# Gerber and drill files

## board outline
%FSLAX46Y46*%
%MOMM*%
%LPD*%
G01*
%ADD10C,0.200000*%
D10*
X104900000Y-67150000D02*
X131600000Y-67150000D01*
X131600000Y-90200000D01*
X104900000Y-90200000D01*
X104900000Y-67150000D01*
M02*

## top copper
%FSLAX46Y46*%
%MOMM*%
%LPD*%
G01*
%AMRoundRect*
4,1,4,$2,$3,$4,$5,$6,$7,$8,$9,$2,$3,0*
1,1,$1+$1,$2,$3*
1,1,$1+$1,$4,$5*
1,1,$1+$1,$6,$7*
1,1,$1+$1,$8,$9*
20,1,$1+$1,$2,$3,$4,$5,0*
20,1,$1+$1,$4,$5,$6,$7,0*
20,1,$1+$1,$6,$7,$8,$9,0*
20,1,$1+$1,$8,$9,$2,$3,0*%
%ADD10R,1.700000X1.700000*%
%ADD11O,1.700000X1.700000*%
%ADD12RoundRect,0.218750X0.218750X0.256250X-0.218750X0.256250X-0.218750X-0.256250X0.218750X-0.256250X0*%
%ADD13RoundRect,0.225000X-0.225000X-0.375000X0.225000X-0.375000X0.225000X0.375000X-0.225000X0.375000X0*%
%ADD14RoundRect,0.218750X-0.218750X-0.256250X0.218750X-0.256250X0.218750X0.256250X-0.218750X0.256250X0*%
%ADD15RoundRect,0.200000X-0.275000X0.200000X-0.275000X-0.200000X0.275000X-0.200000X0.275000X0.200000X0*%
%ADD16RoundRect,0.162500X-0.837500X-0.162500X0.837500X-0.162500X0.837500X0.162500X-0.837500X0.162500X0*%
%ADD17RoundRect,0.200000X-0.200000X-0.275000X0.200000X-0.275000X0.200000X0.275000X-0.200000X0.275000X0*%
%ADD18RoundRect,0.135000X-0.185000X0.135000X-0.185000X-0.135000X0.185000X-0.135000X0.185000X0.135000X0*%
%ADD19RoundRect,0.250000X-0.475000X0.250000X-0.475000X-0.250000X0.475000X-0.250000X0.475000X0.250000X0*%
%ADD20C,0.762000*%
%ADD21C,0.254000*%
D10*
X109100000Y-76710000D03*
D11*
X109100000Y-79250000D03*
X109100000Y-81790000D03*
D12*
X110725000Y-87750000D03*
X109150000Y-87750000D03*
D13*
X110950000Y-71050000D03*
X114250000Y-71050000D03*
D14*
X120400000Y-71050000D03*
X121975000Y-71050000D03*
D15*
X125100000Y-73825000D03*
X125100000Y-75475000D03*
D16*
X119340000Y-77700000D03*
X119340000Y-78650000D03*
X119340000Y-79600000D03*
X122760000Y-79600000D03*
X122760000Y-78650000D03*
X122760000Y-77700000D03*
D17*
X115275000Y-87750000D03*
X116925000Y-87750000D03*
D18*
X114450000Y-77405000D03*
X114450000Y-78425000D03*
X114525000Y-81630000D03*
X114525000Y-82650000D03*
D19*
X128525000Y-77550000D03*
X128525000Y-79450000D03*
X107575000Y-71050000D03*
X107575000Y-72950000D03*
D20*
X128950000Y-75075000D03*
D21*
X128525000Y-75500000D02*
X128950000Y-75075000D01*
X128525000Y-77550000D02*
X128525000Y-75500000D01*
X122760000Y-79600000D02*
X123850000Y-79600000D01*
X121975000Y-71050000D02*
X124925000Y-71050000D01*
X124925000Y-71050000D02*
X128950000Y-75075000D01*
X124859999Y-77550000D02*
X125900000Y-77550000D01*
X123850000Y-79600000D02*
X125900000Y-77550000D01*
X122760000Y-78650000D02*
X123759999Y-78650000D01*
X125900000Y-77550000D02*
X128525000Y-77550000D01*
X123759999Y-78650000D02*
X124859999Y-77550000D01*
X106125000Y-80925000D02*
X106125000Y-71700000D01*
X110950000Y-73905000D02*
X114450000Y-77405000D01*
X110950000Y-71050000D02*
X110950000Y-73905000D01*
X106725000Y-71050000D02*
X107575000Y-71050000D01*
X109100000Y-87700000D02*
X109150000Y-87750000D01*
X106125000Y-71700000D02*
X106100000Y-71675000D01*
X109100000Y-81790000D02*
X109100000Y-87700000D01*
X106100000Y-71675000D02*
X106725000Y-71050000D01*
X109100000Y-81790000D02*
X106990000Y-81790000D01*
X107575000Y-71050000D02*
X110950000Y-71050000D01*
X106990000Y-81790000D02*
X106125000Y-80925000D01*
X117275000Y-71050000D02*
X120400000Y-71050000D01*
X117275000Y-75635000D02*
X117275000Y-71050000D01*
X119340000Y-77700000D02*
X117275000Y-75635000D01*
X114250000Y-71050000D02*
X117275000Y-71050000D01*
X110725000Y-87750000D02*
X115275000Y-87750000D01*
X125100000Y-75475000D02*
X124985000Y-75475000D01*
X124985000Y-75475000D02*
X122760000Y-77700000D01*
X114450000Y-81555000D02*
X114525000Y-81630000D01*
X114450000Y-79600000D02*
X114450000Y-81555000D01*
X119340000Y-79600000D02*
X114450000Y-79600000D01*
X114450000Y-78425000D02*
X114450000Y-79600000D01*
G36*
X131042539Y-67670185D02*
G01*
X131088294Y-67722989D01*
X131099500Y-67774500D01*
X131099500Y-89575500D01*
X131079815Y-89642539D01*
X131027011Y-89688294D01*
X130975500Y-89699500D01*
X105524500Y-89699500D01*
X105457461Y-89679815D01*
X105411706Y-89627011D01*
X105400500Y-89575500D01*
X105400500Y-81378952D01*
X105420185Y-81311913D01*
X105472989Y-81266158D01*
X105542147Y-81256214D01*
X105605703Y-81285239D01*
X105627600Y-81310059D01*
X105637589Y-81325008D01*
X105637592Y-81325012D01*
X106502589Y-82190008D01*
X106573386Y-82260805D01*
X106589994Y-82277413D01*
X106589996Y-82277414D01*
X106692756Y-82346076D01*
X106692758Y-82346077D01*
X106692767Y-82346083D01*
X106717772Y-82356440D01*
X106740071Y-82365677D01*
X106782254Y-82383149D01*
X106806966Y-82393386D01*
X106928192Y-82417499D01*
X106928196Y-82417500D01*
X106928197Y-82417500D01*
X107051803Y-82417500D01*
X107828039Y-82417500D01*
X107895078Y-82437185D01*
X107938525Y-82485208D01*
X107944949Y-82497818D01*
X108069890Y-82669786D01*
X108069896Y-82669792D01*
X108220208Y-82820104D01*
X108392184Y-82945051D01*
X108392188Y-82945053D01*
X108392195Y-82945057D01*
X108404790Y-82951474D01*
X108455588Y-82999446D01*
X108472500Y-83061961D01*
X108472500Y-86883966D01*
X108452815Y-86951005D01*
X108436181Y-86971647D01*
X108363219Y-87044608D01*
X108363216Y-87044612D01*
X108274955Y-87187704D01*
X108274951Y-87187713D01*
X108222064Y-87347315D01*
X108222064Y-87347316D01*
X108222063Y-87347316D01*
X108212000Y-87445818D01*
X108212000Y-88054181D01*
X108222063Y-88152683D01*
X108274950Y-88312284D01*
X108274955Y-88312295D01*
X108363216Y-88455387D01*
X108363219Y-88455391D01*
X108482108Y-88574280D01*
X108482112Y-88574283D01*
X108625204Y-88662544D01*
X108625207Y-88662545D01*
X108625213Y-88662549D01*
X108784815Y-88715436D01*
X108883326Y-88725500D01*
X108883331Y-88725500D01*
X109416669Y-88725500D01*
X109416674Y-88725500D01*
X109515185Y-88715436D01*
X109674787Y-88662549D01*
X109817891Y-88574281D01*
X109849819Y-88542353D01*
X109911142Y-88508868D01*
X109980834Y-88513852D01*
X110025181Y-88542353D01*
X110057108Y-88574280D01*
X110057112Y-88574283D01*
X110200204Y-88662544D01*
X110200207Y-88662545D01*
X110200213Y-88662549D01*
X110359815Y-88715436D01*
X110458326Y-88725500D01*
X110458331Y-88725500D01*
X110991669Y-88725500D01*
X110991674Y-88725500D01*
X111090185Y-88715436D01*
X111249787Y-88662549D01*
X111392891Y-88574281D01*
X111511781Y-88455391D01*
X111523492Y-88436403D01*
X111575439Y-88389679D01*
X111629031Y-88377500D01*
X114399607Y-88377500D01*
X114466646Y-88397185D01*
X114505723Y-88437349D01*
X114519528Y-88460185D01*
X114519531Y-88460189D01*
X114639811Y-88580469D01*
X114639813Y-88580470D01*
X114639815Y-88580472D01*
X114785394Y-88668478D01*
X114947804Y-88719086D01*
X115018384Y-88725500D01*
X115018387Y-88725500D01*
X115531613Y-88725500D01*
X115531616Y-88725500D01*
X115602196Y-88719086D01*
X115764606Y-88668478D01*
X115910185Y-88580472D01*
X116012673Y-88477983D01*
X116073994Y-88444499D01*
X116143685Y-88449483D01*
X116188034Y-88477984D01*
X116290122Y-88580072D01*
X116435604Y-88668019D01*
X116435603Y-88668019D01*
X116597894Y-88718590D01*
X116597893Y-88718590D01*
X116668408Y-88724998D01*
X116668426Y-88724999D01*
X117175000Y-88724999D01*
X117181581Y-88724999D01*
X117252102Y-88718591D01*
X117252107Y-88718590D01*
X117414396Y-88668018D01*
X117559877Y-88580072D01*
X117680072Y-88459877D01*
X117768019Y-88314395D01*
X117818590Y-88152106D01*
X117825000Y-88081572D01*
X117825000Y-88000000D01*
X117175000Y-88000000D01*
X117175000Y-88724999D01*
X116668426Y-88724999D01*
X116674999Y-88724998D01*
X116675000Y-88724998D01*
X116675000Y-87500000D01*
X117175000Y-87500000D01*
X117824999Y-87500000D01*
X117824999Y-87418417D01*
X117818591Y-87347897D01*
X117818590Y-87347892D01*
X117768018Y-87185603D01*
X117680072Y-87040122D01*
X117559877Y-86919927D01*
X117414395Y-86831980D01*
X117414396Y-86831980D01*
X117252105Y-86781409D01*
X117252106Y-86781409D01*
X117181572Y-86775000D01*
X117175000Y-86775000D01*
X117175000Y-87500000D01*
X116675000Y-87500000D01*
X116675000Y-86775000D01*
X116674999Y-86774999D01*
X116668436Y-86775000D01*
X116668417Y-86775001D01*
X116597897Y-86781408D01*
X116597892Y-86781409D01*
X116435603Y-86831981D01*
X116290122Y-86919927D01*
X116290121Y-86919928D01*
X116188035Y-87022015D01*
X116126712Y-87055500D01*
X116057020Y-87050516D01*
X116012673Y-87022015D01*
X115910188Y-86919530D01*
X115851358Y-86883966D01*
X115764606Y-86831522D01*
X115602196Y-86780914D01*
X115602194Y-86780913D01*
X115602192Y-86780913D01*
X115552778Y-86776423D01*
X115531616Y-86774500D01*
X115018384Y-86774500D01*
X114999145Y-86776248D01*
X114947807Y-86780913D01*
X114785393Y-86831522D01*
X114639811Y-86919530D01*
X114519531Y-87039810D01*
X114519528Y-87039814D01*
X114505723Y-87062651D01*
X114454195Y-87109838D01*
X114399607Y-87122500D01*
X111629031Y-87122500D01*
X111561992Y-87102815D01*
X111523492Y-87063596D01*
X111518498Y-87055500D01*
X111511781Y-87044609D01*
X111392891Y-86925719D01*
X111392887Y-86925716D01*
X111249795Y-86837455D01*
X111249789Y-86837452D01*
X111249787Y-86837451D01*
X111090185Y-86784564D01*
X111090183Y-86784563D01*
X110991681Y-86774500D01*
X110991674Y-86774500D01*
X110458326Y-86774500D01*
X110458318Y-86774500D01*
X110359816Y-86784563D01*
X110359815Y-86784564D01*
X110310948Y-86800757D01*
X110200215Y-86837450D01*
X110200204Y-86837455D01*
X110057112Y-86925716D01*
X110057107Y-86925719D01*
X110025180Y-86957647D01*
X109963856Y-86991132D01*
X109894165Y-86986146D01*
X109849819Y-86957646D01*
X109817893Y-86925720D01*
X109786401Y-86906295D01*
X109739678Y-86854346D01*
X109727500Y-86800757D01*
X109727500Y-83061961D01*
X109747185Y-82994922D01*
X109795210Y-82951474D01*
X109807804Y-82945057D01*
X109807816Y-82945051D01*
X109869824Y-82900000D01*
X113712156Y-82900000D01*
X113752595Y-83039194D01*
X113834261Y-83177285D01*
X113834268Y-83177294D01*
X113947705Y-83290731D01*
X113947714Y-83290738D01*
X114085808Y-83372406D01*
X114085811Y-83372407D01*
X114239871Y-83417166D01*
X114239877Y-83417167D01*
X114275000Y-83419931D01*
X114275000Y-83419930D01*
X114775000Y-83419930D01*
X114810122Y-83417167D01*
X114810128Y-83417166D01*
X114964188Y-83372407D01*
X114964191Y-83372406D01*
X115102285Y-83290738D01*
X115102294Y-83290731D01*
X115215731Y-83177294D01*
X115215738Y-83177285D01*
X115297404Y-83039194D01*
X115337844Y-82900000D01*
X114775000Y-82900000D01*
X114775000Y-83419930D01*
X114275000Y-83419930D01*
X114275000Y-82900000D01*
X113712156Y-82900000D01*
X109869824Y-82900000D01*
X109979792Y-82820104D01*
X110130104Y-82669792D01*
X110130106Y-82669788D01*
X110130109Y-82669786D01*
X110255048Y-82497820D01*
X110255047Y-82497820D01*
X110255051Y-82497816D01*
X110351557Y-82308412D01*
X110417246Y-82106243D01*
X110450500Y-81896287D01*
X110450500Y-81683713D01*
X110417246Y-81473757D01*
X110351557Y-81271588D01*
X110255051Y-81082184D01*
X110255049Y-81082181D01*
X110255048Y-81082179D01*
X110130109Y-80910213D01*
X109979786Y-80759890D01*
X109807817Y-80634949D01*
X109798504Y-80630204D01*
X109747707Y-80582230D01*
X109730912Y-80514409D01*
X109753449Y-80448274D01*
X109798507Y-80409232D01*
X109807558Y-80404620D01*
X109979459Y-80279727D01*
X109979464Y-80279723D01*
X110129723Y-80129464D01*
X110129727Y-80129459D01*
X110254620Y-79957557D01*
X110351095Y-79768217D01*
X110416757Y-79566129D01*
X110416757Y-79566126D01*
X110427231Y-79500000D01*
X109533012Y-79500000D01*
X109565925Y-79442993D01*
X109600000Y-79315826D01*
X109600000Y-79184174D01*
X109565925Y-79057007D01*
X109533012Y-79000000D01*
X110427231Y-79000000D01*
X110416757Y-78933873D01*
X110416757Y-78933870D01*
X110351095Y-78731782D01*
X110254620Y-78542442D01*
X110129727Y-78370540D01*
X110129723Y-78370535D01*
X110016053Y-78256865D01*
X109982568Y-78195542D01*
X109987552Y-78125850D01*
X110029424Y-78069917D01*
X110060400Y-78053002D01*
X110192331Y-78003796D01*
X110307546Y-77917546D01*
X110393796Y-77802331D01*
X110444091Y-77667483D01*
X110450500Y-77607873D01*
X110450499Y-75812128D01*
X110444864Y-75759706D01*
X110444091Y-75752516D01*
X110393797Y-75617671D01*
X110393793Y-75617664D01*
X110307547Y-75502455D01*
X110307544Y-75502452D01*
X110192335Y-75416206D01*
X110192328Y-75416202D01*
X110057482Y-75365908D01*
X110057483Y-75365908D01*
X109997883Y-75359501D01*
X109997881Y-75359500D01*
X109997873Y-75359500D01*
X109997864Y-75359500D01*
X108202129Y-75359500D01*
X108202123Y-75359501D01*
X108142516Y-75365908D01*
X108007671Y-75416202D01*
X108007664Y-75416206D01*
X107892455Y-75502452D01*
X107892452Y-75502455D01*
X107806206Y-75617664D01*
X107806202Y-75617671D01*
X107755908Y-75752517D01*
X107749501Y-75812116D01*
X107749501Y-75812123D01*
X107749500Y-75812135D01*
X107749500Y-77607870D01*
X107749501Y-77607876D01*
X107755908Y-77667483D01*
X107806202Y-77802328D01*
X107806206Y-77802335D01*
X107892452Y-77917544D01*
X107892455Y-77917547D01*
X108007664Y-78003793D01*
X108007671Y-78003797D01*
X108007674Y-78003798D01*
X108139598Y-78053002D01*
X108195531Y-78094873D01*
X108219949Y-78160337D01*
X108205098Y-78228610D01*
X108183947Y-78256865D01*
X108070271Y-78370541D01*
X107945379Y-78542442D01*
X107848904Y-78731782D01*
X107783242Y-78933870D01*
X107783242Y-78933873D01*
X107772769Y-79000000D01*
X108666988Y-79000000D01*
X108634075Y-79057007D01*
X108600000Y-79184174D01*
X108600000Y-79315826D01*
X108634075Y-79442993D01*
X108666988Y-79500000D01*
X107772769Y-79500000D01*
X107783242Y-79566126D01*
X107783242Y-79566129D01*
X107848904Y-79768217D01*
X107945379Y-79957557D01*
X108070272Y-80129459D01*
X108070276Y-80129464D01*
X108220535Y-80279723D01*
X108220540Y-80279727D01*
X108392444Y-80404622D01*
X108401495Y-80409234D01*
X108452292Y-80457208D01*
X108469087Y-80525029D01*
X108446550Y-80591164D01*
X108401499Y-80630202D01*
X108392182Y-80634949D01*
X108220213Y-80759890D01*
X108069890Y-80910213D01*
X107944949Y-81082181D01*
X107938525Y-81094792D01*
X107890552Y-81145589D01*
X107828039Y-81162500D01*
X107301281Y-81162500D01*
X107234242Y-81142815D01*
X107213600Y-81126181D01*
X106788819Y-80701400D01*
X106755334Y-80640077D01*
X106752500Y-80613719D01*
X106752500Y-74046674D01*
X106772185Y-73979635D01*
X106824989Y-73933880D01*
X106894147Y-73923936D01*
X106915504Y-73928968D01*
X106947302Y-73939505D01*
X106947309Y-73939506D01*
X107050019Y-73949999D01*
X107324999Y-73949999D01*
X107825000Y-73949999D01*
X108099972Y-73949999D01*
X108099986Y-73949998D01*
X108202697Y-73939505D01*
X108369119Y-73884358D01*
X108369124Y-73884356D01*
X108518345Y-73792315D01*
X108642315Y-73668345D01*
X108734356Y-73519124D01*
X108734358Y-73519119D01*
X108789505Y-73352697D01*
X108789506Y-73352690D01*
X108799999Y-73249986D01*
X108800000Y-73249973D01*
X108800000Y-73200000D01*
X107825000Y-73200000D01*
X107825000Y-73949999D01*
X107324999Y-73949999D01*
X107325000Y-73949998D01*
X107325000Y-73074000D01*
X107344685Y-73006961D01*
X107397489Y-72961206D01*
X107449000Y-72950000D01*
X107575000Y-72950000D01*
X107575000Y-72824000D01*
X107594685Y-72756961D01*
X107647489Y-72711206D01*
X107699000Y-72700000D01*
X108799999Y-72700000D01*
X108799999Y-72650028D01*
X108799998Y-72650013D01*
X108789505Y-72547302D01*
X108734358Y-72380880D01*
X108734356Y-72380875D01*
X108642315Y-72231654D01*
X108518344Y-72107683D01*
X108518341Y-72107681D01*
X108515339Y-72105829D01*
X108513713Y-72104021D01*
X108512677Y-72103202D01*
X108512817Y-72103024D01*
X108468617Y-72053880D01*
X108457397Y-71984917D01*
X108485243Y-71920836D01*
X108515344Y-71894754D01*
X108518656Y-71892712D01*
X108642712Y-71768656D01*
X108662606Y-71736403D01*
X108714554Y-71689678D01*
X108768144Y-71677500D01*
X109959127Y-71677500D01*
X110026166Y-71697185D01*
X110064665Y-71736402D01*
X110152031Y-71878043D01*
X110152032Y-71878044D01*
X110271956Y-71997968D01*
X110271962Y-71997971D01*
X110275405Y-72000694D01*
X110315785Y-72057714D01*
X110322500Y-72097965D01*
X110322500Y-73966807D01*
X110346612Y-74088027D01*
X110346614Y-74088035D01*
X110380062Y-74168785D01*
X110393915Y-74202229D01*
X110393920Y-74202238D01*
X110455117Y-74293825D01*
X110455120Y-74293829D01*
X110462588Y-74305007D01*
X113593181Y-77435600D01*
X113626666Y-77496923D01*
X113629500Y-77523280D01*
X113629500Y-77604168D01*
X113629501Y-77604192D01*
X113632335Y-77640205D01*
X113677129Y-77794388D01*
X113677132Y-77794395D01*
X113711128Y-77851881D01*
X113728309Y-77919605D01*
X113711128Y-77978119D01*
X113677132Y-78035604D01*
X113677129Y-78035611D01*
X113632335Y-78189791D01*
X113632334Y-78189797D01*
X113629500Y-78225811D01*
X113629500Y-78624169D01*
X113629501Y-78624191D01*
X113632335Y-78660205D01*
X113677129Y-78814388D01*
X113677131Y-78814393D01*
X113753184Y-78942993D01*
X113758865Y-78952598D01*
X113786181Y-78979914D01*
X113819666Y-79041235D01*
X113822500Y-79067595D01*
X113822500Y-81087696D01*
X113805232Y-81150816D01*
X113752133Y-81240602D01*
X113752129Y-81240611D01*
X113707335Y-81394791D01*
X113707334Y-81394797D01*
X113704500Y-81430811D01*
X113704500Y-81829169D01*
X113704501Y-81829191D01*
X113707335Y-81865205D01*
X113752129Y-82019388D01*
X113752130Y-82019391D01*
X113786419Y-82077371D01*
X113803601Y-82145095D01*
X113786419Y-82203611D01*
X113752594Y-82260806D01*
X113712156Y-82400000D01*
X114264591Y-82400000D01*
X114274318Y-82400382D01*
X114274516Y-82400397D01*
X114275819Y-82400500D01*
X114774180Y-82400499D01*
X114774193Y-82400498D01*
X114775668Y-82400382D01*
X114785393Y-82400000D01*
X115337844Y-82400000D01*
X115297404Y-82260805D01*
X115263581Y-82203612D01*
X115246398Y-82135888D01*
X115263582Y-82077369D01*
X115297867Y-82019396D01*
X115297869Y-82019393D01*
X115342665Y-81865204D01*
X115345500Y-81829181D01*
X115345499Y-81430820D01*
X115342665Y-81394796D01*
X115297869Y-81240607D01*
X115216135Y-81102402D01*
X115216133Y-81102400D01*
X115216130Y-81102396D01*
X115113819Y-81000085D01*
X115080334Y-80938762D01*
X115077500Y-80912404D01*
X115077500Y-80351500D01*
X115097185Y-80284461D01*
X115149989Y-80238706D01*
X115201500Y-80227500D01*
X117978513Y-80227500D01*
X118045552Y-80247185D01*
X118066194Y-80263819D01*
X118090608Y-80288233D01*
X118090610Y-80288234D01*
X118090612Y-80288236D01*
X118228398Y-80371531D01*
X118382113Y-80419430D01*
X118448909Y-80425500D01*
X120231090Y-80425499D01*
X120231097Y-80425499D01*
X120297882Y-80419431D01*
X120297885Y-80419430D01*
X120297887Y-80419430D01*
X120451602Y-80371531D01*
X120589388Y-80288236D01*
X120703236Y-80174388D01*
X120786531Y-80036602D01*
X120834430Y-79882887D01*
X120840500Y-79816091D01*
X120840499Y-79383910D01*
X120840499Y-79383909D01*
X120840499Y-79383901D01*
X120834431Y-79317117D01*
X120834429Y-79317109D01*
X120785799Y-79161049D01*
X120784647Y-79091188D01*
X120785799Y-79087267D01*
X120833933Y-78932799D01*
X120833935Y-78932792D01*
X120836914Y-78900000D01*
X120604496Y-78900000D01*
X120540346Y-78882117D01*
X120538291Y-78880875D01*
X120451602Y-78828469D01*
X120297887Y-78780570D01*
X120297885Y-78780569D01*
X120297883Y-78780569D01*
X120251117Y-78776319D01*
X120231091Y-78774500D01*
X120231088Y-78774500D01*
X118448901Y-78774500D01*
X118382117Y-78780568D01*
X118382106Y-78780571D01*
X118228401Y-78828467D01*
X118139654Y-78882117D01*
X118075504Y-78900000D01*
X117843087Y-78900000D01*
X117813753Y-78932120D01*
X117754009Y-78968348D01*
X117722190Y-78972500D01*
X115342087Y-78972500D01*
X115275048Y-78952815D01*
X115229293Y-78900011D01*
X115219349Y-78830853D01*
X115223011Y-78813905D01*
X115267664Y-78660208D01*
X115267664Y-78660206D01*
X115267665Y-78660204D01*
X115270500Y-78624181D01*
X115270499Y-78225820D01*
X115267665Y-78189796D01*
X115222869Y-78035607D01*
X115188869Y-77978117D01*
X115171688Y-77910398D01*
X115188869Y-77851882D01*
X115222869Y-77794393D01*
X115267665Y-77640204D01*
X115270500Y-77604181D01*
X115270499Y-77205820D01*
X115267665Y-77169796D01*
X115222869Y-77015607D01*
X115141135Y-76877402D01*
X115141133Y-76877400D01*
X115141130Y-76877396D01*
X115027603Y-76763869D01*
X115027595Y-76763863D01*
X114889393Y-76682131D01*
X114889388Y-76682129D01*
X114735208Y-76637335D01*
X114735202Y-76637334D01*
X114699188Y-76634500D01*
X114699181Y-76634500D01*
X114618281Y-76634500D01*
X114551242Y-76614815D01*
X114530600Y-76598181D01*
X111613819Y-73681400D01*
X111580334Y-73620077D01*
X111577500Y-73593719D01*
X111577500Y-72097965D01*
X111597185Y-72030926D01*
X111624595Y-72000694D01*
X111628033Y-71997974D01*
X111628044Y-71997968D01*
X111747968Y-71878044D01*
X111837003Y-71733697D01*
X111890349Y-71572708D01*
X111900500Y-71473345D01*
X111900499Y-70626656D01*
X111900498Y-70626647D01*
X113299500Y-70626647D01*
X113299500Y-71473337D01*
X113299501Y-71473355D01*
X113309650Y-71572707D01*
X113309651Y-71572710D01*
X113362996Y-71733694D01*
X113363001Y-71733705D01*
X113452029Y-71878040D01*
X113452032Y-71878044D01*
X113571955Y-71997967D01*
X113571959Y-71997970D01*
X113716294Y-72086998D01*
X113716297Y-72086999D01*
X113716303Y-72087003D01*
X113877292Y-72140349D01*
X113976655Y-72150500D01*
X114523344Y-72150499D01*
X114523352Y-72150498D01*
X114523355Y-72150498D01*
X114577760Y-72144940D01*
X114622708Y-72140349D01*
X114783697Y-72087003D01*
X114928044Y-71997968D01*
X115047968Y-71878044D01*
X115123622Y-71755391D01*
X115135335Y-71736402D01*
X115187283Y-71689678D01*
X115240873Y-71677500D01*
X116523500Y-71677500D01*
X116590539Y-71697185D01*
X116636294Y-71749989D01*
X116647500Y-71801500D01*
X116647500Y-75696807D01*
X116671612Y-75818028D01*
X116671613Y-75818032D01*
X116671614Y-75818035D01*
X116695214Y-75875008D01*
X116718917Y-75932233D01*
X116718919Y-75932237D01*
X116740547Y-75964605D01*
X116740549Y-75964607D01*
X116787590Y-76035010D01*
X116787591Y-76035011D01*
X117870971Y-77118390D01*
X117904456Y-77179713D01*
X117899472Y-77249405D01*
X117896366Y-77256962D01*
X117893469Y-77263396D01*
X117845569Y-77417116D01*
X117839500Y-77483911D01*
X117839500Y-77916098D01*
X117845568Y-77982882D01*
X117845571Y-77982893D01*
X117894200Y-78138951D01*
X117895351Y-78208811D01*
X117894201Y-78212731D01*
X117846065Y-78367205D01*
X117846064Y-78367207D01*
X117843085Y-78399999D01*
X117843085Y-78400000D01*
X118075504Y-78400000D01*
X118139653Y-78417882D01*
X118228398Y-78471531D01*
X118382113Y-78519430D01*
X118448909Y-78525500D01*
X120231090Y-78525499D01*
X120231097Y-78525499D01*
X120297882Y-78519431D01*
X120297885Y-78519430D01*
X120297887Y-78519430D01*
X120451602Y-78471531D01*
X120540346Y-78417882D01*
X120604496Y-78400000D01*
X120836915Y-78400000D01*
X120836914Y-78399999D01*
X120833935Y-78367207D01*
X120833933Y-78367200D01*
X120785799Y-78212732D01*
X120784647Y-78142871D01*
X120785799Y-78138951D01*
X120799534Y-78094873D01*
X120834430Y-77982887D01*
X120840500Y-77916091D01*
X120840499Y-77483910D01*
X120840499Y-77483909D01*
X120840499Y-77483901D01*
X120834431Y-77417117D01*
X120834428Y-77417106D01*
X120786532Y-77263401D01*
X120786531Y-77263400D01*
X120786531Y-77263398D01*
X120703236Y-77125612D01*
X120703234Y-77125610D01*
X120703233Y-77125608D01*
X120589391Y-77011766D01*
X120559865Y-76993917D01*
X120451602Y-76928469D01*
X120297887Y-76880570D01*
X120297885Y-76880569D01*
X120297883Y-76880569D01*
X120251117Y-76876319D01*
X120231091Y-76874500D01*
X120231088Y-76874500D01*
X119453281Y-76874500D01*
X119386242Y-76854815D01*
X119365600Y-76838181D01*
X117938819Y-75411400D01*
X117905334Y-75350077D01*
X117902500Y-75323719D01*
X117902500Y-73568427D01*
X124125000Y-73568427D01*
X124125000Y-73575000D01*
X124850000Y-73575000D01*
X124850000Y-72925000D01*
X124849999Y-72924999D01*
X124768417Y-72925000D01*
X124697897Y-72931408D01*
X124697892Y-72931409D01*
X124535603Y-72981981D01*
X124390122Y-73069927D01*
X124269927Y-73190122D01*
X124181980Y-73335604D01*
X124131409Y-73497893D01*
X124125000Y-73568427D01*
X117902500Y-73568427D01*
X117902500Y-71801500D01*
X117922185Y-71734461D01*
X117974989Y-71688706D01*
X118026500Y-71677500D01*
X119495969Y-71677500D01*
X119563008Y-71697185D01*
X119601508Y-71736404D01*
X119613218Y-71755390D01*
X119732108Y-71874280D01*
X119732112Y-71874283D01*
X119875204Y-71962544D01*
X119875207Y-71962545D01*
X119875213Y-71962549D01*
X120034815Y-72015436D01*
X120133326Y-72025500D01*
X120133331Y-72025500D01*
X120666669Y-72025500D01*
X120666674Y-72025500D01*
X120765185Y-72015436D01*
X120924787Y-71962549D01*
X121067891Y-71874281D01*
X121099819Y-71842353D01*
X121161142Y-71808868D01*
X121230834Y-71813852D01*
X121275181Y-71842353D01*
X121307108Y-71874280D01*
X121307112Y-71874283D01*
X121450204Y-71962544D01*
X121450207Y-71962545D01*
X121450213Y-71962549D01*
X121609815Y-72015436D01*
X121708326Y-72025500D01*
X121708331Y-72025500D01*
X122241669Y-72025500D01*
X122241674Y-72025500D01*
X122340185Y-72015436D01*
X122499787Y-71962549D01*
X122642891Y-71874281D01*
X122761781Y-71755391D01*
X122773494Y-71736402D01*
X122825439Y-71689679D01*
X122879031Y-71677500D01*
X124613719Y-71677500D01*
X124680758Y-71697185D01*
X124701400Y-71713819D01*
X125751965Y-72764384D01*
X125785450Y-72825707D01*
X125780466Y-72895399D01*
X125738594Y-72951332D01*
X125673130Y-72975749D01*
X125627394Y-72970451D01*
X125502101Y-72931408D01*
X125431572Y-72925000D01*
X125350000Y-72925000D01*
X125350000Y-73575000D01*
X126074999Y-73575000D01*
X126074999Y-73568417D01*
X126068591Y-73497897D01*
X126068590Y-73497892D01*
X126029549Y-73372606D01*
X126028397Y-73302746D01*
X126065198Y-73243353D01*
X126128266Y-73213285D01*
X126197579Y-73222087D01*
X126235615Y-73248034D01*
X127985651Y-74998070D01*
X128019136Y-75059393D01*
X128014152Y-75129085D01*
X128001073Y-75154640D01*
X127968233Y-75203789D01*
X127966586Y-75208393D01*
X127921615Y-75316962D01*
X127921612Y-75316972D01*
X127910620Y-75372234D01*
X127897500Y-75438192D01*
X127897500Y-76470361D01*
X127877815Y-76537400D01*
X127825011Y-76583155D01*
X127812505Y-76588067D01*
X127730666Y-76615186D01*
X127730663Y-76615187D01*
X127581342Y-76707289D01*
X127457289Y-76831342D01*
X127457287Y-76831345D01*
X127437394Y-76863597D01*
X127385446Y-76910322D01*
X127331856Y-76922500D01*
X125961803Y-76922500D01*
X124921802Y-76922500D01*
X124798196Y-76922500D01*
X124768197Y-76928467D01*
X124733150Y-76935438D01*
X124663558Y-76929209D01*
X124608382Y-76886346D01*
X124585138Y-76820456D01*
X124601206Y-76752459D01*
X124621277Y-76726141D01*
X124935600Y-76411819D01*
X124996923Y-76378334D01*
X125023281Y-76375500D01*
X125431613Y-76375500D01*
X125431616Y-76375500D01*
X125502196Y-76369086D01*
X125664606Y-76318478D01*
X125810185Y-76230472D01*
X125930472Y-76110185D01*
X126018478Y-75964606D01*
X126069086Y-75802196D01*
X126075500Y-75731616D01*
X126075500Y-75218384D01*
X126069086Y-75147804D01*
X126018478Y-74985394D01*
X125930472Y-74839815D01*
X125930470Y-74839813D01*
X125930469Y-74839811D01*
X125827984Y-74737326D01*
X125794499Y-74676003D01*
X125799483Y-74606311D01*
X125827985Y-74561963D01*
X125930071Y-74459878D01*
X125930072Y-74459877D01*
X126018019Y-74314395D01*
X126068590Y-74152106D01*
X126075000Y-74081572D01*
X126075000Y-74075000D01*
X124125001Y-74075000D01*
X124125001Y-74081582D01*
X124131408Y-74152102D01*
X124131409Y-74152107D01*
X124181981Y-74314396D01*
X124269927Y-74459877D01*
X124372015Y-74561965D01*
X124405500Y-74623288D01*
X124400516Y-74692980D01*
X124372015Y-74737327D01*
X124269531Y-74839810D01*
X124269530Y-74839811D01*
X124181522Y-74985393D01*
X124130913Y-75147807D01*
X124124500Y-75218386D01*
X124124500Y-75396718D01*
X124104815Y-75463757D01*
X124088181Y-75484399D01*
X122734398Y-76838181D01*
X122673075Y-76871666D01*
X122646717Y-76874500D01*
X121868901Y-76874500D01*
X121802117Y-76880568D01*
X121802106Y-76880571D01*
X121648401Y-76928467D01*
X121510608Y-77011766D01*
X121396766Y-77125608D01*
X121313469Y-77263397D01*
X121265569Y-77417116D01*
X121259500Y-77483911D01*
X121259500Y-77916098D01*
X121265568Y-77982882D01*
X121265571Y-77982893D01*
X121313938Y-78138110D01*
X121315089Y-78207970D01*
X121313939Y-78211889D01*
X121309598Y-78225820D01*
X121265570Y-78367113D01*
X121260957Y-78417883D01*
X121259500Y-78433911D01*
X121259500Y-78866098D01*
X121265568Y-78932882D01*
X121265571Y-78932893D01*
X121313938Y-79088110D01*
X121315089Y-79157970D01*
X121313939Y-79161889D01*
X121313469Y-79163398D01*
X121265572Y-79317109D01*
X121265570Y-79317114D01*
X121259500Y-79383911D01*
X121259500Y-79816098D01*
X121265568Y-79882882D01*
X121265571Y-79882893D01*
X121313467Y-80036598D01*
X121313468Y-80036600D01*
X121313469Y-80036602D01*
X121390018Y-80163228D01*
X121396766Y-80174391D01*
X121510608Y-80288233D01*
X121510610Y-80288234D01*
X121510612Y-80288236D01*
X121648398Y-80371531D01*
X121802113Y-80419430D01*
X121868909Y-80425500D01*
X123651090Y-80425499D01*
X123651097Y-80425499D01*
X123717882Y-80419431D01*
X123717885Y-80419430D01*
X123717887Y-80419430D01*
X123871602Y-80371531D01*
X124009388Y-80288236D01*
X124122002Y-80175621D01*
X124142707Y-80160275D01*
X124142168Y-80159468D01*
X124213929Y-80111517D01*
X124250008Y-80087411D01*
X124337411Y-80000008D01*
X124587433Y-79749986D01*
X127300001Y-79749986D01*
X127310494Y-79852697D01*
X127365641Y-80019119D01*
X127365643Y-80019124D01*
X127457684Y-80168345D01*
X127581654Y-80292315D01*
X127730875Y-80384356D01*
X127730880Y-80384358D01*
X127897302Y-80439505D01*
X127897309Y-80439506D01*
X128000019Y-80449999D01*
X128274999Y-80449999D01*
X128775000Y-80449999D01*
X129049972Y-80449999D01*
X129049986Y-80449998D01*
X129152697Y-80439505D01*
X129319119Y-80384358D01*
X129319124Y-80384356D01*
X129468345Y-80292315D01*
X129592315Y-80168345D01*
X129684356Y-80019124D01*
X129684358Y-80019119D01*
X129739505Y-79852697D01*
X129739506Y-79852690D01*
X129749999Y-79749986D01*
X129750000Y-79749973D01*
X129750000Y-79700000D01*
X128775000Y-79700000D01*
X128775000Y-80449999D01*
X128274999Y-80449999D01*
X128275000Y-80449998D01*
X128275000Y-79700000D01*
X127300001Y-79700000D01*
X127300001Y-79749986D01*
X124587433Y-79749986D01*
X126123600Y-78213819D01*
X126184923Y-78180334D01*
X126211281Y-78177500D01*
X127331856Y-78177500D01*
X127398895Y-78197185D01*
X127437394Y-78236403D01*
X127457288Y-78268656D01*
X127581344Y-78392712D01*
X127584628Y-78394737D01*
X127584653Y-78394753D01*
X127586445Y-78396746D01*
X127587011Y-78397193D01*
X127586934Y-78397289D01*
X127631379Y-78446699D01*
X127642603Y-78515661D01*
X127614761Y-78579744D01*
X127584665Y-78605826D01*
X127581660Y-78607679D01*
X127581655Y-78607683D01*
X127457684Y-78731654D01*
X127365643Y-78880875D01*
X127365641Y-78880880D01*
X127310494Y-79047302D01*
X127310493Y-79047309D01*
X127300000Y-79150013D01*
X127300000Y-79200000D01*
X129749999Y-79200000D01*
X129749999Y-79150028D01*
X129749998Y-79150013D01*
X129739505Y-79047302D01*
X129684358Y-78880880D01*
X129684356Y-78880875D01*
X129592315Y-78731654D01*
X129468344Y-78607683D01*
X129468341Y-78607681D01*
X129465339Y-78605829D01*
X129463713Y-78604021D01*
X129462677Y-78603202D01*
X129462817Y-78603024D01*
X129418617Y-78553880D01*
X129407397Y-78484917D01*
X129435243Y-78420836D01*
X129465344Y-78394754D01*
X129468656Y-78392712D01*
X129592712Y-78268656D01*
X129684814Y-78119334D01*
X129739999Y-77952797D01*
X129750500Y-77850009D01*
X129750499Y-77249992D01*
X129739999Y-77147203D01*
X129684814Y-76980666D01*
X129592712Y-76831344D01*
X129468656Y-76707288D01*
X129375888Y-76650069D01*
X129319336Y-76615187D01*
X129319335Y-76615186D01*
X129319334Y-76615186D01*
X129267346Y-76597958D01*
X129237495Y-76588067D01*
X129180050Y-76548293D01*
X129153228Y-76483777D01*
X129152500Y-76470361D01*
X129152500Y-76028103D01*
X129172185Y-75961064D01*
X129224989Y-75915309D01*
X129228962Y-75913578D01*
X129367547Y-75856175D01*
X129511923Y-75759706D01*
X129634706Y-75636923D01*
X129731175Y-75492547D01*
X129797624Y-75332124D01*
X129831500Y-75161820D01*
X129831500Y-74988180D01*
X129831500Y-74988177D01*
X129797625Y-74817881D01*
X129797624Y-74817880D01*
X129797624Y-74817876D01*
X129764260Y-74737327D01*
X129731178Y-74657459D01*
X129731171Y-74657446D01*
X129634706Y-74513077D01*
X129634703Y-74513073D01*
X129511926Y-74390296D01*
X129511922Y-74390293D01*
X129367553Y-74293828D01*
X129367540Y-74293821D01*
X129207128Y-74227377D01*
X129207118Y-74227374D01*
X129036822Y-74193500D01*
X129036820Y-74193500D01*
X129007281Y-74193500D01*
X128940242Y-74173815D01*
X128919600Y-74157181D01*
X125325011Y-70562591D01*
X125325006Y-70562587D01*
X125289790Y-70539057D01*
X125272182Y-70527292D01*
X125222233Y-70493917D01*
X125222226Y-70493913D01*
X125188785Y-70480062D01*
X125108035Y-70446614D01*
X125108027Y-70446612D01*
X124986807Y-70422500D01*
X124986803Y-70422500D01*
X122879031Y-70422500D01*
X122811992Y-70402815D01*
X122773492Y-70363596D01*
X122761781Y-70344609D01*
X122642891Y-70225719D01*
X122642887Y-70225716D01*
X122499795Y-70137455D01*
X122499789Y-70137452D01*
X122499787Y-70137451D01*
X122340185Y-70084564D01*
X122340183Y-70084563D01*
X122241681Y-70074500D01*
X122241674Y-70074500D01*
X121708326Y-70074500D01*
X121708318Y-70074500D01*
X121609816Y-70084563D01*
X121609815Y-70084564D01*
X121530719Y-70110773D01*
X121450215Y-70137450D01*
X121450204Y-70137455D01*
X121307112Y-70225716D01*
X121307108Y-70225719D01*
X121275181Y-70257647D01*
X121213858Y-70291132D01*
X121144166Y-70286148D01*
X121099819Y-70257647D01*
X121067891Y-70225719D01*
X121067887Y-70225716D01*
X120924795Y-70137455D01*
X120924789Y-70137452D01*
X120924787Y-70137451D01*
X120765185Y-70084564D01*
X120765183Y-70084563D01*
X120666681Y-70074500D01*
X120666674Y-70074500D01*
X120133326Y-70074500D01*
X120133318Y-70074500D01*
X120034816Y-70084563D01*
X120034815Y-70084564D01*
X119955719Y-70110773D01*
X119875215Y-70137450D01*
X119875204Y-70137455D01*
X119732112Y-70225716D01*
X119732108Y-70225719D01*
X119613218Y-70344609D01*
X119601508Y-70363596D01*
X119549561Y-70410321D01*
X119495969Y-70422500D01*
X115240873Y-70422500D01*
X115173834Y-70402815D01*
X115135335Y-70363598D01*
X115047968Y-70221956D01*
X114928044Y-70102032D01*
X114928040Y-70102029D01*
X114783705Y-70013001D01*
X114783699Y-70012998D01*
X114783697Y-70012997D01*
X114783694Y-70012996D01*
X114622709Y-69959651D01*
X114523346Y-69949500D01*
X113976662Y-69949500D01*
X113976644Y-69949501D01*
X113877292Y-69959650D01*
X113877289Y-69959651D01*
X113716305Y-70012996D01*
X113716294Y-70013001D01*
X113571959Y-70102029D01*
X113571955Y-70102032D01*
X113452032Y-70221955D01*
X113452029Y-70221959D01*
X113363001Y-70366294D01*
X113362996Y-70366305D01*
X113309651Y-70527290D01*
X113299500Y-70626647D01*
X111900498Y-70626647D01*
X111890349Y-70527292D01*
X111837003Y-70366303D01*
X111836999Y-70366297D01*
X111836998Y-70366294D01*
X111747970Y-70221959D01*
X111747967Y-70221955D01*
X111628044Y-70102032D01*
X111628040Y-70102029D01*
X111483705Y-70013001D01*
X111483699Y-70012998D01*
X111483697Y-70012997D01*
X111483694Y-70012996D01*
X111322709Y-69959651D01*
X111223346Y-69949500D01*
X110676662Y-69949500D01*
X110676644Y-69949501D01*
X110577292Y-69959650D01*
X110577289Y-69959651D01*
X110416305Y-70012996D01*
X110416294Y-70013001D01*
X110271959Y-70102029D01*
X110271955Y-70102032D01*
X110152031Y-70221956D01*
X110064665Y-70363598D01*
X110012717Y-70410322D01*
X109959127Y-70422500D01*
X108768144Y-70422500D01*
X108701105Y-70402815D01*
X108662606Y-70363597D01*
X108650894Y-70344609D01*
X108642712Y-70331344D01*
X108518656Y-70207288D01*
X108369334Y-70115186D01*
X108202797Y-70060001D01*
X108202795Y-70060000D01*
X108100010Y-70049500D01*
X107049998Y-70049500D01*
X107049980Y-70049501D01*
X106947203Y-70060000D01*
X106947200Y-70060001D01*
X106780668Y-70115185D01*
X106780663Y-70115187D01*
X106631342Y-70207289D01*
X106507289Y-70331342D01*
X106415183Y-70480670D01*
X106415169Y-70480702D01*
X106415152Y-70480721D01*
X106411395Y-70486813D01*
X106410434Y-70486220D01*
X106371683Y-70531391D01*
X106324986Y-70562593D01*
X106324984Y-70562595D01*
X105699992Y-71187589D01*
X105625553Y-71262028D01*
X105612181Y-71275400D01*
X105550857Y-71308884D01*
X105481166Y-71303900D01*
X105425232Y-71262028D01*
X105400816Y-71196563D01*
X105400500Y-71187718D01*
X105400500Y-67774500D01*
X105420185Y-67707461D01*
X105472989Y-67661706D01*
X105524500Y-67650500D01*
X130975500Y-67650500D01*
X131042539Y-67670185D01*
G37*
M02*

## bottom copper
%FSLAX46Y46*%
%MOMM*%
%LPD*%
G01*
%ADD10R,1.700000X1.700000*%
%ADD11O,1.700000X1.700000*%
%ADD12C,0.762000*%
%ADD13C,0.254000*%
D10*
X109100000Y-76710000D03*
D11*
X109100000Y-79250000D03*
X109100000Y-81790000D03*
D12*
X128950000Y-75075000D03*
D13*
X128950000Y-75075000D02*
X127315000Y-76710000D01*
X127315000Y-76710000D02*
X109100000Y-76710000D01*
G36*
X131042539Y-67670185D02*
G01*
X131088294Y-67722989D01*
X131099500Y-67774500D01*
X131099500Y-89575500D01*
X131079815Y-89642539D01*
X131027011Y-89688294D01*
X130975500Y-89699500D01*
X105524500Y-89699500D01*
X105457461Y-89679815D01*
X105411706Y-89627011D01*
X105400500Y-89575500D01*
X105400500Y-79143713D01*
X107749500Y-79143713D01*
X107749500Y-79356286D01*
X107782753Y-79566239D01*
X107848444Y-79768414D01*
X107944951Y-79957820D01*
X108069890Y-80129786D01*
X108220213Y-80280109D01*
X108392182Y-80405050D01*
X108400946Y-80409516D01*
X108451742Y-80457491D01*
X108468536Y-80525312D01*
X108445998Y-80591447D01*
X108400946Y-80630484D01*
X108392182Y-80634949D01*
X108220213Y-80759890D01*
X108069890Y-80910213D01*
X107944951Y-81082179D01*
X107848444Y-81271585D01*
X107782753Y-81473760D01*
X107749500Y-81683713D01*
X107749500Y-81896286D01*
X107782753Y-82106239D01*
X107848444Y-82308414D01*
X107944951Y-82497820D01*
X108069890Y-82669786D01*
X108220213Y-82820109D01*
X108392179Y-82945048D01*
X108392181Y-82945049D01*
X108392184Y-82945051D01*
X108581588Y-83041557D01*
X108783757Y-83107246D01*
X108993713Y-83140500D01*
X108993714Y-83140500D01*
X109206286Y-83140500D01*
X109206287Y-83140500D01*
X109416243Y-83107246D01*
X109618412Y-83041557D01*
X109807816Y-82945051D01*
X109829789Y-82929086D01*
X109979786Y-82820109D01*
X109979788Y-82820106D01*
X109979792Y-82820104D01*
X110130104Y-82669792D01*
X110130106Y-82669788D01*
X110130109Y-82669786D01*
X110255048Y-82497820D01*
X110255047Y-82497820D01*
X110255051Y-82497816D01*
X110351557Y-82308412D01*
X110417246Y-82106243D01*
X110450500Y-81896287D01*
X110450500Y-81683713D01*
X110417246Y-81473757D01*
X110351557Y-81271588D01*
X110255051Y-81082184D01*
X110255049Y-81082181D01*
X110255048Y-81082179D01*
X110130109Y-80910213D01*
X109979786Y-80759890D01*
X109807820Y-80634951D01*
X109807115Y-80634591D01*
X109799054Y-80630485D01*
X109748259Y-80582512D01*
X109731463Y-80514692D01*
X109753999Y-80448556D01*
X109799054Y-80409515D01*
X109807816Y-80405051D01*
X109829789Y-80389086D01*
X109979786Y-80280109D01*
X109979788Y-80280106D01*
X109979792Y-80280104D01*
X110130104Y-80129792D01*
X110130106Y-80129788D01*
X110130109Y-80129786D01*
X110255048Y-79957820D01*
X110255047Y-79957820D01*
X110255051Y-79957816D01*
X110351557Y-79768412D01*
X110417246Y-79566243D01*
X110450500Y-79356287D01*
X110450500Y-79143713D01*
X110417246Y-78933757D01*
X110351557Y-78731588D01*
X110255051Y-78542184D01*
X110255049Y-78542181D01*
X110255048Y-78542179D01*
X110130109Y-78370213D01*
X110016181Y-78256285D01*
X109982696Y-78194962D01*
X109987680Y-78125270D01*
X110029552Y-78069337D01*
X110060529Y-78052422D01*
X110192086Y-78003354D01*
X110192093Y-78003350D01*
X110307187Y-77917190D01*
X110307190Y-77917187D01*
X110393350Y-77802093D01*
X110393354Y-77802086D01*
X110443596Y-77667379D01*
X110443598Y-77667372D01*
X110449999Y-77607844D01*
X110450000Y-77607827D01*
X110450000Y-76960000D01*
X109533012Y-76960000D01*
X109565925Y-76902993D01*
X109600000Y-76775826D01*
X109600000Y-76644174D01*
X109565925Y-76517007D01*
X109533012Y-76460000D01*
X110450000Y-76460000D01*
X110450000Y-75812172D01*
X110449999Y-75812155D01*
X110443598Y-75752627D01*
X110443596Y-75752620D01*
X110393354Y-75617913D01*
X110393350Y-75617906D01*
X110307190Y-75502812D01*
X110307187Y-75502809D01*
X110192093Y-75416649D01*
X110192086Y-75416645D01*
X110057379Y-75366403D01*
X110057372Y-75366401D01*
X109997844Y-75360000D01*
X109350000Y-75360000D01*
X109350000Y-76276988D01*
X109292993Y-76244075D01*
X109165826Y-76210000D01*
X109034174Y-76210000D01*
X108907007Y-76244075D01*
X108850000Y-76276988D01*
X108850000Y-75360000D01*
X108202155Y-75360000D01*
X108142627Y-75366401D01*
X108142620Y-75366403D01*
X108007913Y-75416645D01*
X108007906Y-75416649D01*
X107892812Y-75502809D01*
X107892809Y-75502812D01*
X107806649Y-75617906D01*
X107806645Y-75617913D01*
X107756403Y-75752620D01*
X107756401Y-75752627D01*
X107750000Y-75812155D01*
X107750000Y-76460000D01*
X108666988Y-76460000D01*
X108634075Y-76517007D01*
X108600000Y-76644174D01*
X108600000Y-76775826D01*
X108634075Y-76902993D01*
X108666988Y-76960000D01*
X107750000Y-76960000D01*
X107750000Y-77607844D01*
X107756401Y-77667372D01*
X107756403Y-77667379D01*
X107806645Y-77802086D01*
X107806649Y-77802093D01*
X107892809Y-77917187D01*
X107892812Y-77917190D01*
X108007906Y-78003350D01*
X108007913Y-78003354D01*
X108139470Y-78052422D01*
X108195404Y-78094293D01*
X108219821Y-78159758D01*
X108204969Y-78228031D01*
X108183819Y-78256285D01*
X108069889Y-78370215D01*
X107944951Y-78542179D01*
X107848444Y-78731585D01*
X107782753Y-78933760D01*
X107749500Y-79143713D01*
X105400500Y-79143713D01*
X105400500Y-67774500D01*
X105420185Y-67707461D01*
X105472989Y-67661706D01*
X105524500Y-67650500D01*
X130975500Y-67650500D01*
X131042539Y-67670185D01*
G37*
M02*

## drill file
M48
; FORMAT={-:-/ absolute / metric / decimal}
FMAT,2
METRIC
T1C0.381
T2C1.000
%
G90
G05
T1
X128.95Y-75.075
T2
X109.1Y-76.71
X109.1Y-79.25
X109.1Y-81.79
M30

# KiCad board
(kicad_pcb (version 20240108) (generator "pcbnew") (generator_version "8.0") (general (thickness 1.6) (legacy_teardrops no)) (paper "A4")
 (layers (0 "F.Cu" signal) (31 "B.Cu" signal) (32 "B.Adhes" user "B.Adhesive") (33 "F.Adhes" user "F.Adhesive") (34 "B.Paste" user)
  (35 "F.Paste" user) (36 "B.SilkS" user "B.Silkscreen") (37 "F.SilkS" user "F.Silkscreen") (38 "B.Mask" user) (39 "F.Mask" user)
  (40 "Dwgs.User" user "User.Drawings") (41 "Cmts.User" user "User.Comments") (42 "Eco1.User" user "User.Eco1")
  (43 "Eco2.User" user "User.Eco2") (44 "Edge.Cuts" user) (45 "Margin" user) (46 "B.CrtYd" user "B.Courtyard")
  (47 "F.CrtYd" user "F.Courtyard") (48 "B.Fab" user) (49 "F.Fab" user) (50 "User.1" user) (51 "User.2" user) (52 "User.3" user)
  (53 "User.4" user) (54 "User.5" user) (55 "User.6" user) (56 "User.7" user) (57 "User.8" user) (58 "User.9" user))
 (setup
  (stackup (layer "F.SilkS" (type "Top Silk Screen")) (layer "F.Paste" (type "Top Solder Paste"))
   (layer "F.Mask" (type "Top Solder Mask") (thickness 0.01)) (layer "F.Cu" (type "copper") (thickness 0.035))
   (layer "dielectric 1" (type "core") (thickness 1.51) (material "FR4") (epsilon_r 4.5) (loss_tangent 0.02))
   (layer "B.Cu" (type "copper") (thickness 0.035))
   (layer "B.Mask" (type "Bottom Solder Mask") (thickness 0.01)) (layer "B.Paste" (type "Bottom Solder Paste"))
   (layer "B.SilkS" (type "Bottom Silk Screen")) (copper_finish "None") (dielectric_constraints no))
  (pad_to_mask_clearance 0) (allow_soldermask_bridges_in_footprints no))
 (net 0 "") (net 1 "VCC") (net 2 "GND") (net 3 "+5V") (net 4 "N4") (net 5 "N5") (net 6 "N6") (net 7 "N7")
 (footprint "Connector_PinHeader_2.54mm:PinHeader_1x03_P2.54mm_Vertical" (layer "F.Cu") (at 109.1 76.71)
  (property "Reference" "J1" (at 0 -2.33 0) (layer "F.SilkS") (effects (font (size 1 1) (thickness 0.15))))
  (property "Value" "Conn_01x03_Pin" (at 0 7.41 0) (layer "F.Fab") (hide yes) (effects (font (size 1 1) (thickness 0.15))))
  (pad "1" thru_hole rect (at 0 0) (size 1.7 1.7) (drill 1) (layers "*.Cu" "*.Mask") (remove_unused_layers no) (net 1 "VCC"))
  (pad "2" thru_hole oval (at 0 2.54) (size 1.7 1.7) (drill 1) (layers "*.Cu" "*.Mask") (remove_unused_layers no) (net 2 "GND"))
  (pad "3" thru_hole oval (at 0 5.08) (size 1.7 1.7) (drill 1) (layers "*.Cu" "*.Mask") (remove_unused_layers no) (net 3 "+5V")))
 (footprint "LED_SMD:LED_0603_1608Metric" (layer "F.Cu") (at 109.9375 87.75 180)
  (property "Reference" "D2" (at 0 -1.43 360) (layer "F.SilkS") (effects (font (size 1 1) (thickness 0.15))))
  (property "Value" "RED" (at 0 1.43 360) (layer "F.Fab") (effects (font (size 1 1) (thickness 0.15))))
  (pad "1" smd roundrect (at -0.7875 0 180) (size 0.875 0.95) (layers "F.Cu" "F.Paste" "F.Mask") (roundrect_rratio 0.25) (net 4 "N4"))
  (pad "2" smd roundrect (at 0.7875 0 180) (size 0.875 0.95) (layers "F.Cu" "F.Paste" "F.Mask") (roundrect_rratio 0.25) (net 3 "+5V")))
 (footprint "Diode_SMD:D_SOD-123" (layer "F.Cu") (at 112.6 71.05)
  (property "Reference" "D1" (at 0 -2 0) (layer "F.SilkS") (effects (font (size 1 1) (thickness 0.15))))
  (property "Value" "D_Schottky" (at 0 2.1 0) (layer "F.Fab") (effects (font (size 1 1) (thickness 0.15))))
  (pad "1" smd roundrect (at -1.65 0) (size 0.9 1.2) (layers "F.Cu" "F.Paste" "F.Mask") (roundrect_rratio 0.25) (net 3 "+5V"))
  (pad "2" smd roundrect (at 1.65 0) (size 0.9 1.2) (layers "F.Cu" "F.Paste" "F.Mask") (roundrect_rratio 0.25) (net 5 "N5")))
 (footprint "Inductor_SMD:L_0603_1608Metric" (layer "F.Cu") (at 121.1875 71.05)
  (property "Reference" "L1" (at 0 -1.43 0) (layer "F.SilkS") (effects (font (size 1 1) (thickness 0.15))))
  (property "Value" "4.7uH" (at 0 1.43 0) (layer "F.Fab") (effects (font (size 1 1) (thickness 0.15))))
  (pad "1" smd roundrect (at -0.7875 0) (size 0.875 0.95) (layers "F.Cu" "F.Paste" "F.Mask") (roundrect_rratio 0.25) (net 5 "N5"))
  (pad "2" smd roundrect (at 0.7875 0) (size 0.875 0.95) (layers "F.Cu" "F.Paste" "F.Mask") (roundrect_rratio 0.25) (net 1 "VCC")))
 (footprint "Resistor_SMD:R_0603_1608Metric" (layer "F.Cu") (at 125.1 74.65 -90)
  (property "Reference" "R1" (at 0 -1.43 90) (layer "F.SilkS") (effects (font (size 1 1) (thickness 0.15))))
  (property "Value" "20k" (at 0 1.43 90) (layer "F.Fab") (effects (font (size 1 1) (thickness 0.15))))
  (pad "1" smd roundrect (at -0.825 0 270) (size 0.8 0.95) (layers "F.Cu" "F.Paste" "F.Mask") (roundrect_rratio 0.25) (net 2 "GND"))
  (pad "2" smd roundrect (at 0.825 0 270) (size 0.8 0.95) (layers "F.Cu" "F.Paste" "F.Mask") (roundrect_rratio 0.25) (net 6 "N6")))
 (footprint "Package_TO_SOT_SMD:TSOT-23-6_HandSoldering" (layer "F.Cu") (at 121.05 78.65)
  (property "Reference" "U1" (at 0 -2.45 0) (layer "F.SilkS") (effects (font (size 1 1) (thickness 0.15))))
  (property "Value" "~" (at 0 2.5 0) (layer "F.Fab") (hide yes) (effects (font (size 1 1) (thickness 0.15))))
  (pad "1" smd roundrect (at -1.71 -0.95) (size 2 0.65) (layers "F.Cu" "F.Paste" "F.Mask") (roundrect_rratio 0.25) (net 5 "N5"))
  (pad "2" smd roundrect (at -1.71 0) (size 2 0.65) (layers "F.Cu" "F.Paste" "F.Mask") (roundrect_rratio 0.25) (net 2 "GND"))
  (pad "3" smd roundrect (at -1.71 0.95) (size 2 0.65) (layers "F.Cu" "F.Paste" "F.Mask") (roundrect_rratio 0.25) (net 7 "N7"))
  (pad "4" smd roundrect (at 1.71 0.95) (size 2 0.65) (layers "F.Cu" "F.Paste" "F.Mask") (roundrect_rratio 0.25) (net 1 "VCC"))
  (pad "5" smd roundrect (at 1.71 0) (size 2 0.65) (layers "F.Cu" "F.Paste" "F.Mask") (roundrect_rratio 0.25) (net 1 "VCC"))
  (pad "6" smd roundrect (at 1.71 -0.95) (size 2 0.65) (layers "F.Cu" "F.Paste" "F.Mask") (roundrect_rratio 0.25) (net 6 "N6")))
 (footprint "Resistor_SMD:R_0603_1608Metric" (layer "F.Cu") (at 116.1 87.75)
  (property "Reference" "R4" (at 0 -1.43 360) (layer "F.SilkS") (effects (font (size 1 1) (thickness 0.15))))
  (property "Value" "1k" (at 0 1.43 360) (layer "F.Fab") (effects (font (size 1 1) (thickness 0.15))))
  (pad "1" smd roundrect (at -0.825 0) (size 0.8 0.95) (layers "F.Cu" "F.Paste" "F.Mask") (roundrect_rratio 0.25) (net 4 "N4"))
  (pad "2" smd roundrect (at 0.825 0) (size 0.8 0.95) (layers "F.Cu" "F.Paste" "F.Mask") (roundrect_rratio 0.25) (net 2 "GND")))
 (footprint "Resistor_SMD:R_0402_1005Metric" (layer "F.Cu") (at 114.45 77.915 -90)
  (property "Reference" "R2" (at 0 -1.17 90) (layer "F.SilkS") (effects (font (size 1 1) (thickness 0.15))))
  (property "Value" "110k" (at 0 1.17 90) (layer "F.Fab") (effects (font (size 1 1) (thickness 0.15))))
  (pad "1" smd roundrect (at -0.51 0 270) (size 0.54 0.64) (layers "F.Cu" "F.Paste" "F.Mask") (roundrect_rratio 0.25) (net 3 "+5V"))
  (pad "2" smd roundrect (at 0.51 0 270) (size 0.54 0.64) (layers "F.Cu" "F.Paste" "F.Mask") (roundrect_rratio 0.25) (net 7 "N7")))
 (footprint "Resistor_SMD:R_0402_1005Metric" (layer "F.Cu") (at 114.525 82.14 -90)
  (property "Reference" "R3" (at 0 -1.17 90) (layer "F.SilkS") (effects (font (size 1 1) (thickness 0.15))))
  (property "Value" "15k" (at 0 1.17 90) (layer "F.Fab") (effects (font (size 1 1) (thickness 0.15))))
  (pad "1" smd roundrect (at -0.51 0 270) (size 0.54 0.64) (layers "F.Cu" "F.Paste" "F.Mask") (roundrect_rratio 0.25) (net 7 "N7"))
  (pad "2" smd roundrect (at 0.51 0 270) (size 0.54 0.64) (layers "F.Cu" "F.Paste" "F.Mask") (roundrect_rratio 0.25) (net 2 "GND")))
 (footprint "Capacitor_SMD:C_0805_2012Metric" (layer "F.Cu") (at 128.525 78.5 -90)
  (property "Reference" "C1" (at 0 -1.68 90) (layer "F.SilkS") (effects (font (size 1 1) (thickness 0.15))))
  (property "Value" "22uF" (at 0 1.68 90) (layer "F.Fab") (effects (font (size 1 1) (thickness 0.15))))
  (pad "1" smd roundrect (at -0.95 0 270) (size 1 1.45) (layers "F.Cu" "F.Paste" "F.Mask") (roundrect_rratio 0.25) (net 1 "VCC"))
  (pad "2" smd roundrect (at 0.95 0 270) (size 1 1.45) (layers "F.Cu" "F.Paste" "F.Mask") (roundrect_rratio 0.25) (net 2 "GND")))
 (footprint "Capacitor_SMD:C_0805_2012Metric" (layer "F.Cu") (at 107.575 72 -90)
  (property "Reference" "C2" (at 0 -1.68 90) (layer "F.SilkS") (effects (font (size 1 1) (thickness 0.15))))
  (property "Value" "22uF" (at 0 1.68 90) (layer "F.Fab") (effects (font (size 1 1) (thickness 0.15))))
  (pad "1" smd roundrect (at -0.95 0 270) (size 1 1.45) (layers "F.Cu" "F.Paste" "F.Mask") (roundrect_rratio 0.25) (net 3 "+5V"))
  (pad "2" smd roundrect (at 0.95 0 270) (size 1 1.45) (layers "F.Cu" "F.Paste" "F.Mask") (roundrect_rratio 0.25) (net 2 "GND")))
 (gr_rect (start 104.9 67.15) (end 131.6 90.2) (stroke (width 0.2) (type default)) (fill none) (layer "Edge.Cuts"))
 (segment (start 128.525 75.5) (end 128.95 75.075) (width 0.254) (layer "F.Cu") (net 1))
 (segment (start 128.525 77.55) (end 128.525 75.5) (width 0.254) (layer "F.Cu") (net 1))
 (segment (start 122.76 79.6) (end 123.85 79.6) (width 0.254) (layer "F.Cu") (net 1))
 (segment (start 121.975 71.05) (end 124.925 71.05) (width 0.254) (layer "F.Cu") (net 1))
 (segment (start 124.925 71.05) (end 128.95 75.075) (width 0.254) (layer "F.Cu") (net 1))
 (segment (start 124.859999 77.55) (end 125.9 77.55) (width 0.254) (layer "F.Cu") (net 1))
 (segment (start 123.85 79.6) (end 125.9 77.55) (width 0.254) (layer "F.Cu") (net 1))
 (segment (start 122.76 78.65) (end 123.759999 78.65) (width 0.254) (layer "F.Cu") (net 1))
 (segment (start 125.9 77.55) (end 128.525 77.55) (width 0.254) (layer "F.Cu") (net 1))
 (segment (start 123.759999 78.65) (end 124.859999 77.55) (width 0.254) (layer "F.Cu") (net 1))
 (via (at 128.95 75.075) (size 0.762) (drill 0.381) (layers "F.Cu" "B.Cu") (free yes) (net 1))
 (segment (start 128.95 75.075) (end 127.315 76.71) (width 0.254) (layer "B.Cu") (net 1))
 (segment (start 127.315 76.71) (end 109.1 76.71) (width 0.254) (layer "B.Cu") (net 1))
 (segment (start 106.125 80.925) (end 106.125 71.7) (width 0.254) (layer "F.Cu") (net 3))
 (segment (start 110.95 73.905) (end 114.45 77.405) (width 0.254) (layer "F.Cu") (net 3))
 (segment (start 110.95 71.05) (end 110.95 73.905) (width 0.254) (layer "F.Cu") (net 3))
 (segment (start 106.725 71.05) (end 107.575 71.05) (width 0.254) (layer "F.Cu") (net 3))
 (segment (start 109.1 87.7) (end 109.15 87.75) (width 0.254) (layer "F.Cu") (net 3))
 (segment (start 106.125 71.7) (end 106.1 71.675) (width 0.254) (layer "F.Cu") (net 3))
 (segment (start 109.1 81.79) (end 109.1 87.7) (width 0.254) (layer "F.Cu") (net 3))
 (segment (start 106.1 71.675) (end 106.725 71.05) (width 0.254) (layer "F.Cu") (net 3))
 (segment (start 109.1 81.79) (end 106.99 81.79) (width 0.254) (layer "F.Cu") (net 3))
 (segment (start 107.575 71.05) (end 110.95 71.05) (width 0.254) (layer "F.Cu") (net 3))
 (segment (start 106.99 81.79) (end 106.125 80.925) (width 0.254) (layer "F.Cu") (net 3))
 (segment (start 117.275 71.05) (end 120.4 71.05) (width 0.254) (layer "F.Cu") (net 5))
 (segment (start 117.275 75.635) (end 117.275 71.05) (width 0.254) (layer "F.Cu") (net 5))
 (segment (start 119.34 77.7) (end 117.275 75.635) (width 0.254) (layer "F.Cu") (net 5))
 (segment (start 114.25 71.05) (end 117.275 71.05) (width 0.254) (layer "F.Cu") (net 5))
 (segment (start 110.725 87.75) (end 115.275 87.75) (width 0.254) (layer "F.Cu") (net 4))
 (segment (start 125.1 75.475) (end 124.985 75.475) (width 0.254) (layer "F.Cu") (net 6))
 (segment (start 124.985 75.475) (end 122.76 77.7) (width 0.254) (layer "F.Cu") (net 6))
 (segment (start 114.45 81.555) (end 114.525 81.63) (width 0.254) (layer "F.Cu") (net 7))
 (segment (start 114.45 79.6) (end 114.45 81.555) (width 0.254) (layer "F.Cu") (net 7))
 (segment (start 119.34 79.6) (end 114.45 79.6) (width 0.254) (layer "F.Cu") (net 7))
 (segment (start 114.45 78.425) (end 114.45 79.6) (width 0.254) (layer "F.Cu") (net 7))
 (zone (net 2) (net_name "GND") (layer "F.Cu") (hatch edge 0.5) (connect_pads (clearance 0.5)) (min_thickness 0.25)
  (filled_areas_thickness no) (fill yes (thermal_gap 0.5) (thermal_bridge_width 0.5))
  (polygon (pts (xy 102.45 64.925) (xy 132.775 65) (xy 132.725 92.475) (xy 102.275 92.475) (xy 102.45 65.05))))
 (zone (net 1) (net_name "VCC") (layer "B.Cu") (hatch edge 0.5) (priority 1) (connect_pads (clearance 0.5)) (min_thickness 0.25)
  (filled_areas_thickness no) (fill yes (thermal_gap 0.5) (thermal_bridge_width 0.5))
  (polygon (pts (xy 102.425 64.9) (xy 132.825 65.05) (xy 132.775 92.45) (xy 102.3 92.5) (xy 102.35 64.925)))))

